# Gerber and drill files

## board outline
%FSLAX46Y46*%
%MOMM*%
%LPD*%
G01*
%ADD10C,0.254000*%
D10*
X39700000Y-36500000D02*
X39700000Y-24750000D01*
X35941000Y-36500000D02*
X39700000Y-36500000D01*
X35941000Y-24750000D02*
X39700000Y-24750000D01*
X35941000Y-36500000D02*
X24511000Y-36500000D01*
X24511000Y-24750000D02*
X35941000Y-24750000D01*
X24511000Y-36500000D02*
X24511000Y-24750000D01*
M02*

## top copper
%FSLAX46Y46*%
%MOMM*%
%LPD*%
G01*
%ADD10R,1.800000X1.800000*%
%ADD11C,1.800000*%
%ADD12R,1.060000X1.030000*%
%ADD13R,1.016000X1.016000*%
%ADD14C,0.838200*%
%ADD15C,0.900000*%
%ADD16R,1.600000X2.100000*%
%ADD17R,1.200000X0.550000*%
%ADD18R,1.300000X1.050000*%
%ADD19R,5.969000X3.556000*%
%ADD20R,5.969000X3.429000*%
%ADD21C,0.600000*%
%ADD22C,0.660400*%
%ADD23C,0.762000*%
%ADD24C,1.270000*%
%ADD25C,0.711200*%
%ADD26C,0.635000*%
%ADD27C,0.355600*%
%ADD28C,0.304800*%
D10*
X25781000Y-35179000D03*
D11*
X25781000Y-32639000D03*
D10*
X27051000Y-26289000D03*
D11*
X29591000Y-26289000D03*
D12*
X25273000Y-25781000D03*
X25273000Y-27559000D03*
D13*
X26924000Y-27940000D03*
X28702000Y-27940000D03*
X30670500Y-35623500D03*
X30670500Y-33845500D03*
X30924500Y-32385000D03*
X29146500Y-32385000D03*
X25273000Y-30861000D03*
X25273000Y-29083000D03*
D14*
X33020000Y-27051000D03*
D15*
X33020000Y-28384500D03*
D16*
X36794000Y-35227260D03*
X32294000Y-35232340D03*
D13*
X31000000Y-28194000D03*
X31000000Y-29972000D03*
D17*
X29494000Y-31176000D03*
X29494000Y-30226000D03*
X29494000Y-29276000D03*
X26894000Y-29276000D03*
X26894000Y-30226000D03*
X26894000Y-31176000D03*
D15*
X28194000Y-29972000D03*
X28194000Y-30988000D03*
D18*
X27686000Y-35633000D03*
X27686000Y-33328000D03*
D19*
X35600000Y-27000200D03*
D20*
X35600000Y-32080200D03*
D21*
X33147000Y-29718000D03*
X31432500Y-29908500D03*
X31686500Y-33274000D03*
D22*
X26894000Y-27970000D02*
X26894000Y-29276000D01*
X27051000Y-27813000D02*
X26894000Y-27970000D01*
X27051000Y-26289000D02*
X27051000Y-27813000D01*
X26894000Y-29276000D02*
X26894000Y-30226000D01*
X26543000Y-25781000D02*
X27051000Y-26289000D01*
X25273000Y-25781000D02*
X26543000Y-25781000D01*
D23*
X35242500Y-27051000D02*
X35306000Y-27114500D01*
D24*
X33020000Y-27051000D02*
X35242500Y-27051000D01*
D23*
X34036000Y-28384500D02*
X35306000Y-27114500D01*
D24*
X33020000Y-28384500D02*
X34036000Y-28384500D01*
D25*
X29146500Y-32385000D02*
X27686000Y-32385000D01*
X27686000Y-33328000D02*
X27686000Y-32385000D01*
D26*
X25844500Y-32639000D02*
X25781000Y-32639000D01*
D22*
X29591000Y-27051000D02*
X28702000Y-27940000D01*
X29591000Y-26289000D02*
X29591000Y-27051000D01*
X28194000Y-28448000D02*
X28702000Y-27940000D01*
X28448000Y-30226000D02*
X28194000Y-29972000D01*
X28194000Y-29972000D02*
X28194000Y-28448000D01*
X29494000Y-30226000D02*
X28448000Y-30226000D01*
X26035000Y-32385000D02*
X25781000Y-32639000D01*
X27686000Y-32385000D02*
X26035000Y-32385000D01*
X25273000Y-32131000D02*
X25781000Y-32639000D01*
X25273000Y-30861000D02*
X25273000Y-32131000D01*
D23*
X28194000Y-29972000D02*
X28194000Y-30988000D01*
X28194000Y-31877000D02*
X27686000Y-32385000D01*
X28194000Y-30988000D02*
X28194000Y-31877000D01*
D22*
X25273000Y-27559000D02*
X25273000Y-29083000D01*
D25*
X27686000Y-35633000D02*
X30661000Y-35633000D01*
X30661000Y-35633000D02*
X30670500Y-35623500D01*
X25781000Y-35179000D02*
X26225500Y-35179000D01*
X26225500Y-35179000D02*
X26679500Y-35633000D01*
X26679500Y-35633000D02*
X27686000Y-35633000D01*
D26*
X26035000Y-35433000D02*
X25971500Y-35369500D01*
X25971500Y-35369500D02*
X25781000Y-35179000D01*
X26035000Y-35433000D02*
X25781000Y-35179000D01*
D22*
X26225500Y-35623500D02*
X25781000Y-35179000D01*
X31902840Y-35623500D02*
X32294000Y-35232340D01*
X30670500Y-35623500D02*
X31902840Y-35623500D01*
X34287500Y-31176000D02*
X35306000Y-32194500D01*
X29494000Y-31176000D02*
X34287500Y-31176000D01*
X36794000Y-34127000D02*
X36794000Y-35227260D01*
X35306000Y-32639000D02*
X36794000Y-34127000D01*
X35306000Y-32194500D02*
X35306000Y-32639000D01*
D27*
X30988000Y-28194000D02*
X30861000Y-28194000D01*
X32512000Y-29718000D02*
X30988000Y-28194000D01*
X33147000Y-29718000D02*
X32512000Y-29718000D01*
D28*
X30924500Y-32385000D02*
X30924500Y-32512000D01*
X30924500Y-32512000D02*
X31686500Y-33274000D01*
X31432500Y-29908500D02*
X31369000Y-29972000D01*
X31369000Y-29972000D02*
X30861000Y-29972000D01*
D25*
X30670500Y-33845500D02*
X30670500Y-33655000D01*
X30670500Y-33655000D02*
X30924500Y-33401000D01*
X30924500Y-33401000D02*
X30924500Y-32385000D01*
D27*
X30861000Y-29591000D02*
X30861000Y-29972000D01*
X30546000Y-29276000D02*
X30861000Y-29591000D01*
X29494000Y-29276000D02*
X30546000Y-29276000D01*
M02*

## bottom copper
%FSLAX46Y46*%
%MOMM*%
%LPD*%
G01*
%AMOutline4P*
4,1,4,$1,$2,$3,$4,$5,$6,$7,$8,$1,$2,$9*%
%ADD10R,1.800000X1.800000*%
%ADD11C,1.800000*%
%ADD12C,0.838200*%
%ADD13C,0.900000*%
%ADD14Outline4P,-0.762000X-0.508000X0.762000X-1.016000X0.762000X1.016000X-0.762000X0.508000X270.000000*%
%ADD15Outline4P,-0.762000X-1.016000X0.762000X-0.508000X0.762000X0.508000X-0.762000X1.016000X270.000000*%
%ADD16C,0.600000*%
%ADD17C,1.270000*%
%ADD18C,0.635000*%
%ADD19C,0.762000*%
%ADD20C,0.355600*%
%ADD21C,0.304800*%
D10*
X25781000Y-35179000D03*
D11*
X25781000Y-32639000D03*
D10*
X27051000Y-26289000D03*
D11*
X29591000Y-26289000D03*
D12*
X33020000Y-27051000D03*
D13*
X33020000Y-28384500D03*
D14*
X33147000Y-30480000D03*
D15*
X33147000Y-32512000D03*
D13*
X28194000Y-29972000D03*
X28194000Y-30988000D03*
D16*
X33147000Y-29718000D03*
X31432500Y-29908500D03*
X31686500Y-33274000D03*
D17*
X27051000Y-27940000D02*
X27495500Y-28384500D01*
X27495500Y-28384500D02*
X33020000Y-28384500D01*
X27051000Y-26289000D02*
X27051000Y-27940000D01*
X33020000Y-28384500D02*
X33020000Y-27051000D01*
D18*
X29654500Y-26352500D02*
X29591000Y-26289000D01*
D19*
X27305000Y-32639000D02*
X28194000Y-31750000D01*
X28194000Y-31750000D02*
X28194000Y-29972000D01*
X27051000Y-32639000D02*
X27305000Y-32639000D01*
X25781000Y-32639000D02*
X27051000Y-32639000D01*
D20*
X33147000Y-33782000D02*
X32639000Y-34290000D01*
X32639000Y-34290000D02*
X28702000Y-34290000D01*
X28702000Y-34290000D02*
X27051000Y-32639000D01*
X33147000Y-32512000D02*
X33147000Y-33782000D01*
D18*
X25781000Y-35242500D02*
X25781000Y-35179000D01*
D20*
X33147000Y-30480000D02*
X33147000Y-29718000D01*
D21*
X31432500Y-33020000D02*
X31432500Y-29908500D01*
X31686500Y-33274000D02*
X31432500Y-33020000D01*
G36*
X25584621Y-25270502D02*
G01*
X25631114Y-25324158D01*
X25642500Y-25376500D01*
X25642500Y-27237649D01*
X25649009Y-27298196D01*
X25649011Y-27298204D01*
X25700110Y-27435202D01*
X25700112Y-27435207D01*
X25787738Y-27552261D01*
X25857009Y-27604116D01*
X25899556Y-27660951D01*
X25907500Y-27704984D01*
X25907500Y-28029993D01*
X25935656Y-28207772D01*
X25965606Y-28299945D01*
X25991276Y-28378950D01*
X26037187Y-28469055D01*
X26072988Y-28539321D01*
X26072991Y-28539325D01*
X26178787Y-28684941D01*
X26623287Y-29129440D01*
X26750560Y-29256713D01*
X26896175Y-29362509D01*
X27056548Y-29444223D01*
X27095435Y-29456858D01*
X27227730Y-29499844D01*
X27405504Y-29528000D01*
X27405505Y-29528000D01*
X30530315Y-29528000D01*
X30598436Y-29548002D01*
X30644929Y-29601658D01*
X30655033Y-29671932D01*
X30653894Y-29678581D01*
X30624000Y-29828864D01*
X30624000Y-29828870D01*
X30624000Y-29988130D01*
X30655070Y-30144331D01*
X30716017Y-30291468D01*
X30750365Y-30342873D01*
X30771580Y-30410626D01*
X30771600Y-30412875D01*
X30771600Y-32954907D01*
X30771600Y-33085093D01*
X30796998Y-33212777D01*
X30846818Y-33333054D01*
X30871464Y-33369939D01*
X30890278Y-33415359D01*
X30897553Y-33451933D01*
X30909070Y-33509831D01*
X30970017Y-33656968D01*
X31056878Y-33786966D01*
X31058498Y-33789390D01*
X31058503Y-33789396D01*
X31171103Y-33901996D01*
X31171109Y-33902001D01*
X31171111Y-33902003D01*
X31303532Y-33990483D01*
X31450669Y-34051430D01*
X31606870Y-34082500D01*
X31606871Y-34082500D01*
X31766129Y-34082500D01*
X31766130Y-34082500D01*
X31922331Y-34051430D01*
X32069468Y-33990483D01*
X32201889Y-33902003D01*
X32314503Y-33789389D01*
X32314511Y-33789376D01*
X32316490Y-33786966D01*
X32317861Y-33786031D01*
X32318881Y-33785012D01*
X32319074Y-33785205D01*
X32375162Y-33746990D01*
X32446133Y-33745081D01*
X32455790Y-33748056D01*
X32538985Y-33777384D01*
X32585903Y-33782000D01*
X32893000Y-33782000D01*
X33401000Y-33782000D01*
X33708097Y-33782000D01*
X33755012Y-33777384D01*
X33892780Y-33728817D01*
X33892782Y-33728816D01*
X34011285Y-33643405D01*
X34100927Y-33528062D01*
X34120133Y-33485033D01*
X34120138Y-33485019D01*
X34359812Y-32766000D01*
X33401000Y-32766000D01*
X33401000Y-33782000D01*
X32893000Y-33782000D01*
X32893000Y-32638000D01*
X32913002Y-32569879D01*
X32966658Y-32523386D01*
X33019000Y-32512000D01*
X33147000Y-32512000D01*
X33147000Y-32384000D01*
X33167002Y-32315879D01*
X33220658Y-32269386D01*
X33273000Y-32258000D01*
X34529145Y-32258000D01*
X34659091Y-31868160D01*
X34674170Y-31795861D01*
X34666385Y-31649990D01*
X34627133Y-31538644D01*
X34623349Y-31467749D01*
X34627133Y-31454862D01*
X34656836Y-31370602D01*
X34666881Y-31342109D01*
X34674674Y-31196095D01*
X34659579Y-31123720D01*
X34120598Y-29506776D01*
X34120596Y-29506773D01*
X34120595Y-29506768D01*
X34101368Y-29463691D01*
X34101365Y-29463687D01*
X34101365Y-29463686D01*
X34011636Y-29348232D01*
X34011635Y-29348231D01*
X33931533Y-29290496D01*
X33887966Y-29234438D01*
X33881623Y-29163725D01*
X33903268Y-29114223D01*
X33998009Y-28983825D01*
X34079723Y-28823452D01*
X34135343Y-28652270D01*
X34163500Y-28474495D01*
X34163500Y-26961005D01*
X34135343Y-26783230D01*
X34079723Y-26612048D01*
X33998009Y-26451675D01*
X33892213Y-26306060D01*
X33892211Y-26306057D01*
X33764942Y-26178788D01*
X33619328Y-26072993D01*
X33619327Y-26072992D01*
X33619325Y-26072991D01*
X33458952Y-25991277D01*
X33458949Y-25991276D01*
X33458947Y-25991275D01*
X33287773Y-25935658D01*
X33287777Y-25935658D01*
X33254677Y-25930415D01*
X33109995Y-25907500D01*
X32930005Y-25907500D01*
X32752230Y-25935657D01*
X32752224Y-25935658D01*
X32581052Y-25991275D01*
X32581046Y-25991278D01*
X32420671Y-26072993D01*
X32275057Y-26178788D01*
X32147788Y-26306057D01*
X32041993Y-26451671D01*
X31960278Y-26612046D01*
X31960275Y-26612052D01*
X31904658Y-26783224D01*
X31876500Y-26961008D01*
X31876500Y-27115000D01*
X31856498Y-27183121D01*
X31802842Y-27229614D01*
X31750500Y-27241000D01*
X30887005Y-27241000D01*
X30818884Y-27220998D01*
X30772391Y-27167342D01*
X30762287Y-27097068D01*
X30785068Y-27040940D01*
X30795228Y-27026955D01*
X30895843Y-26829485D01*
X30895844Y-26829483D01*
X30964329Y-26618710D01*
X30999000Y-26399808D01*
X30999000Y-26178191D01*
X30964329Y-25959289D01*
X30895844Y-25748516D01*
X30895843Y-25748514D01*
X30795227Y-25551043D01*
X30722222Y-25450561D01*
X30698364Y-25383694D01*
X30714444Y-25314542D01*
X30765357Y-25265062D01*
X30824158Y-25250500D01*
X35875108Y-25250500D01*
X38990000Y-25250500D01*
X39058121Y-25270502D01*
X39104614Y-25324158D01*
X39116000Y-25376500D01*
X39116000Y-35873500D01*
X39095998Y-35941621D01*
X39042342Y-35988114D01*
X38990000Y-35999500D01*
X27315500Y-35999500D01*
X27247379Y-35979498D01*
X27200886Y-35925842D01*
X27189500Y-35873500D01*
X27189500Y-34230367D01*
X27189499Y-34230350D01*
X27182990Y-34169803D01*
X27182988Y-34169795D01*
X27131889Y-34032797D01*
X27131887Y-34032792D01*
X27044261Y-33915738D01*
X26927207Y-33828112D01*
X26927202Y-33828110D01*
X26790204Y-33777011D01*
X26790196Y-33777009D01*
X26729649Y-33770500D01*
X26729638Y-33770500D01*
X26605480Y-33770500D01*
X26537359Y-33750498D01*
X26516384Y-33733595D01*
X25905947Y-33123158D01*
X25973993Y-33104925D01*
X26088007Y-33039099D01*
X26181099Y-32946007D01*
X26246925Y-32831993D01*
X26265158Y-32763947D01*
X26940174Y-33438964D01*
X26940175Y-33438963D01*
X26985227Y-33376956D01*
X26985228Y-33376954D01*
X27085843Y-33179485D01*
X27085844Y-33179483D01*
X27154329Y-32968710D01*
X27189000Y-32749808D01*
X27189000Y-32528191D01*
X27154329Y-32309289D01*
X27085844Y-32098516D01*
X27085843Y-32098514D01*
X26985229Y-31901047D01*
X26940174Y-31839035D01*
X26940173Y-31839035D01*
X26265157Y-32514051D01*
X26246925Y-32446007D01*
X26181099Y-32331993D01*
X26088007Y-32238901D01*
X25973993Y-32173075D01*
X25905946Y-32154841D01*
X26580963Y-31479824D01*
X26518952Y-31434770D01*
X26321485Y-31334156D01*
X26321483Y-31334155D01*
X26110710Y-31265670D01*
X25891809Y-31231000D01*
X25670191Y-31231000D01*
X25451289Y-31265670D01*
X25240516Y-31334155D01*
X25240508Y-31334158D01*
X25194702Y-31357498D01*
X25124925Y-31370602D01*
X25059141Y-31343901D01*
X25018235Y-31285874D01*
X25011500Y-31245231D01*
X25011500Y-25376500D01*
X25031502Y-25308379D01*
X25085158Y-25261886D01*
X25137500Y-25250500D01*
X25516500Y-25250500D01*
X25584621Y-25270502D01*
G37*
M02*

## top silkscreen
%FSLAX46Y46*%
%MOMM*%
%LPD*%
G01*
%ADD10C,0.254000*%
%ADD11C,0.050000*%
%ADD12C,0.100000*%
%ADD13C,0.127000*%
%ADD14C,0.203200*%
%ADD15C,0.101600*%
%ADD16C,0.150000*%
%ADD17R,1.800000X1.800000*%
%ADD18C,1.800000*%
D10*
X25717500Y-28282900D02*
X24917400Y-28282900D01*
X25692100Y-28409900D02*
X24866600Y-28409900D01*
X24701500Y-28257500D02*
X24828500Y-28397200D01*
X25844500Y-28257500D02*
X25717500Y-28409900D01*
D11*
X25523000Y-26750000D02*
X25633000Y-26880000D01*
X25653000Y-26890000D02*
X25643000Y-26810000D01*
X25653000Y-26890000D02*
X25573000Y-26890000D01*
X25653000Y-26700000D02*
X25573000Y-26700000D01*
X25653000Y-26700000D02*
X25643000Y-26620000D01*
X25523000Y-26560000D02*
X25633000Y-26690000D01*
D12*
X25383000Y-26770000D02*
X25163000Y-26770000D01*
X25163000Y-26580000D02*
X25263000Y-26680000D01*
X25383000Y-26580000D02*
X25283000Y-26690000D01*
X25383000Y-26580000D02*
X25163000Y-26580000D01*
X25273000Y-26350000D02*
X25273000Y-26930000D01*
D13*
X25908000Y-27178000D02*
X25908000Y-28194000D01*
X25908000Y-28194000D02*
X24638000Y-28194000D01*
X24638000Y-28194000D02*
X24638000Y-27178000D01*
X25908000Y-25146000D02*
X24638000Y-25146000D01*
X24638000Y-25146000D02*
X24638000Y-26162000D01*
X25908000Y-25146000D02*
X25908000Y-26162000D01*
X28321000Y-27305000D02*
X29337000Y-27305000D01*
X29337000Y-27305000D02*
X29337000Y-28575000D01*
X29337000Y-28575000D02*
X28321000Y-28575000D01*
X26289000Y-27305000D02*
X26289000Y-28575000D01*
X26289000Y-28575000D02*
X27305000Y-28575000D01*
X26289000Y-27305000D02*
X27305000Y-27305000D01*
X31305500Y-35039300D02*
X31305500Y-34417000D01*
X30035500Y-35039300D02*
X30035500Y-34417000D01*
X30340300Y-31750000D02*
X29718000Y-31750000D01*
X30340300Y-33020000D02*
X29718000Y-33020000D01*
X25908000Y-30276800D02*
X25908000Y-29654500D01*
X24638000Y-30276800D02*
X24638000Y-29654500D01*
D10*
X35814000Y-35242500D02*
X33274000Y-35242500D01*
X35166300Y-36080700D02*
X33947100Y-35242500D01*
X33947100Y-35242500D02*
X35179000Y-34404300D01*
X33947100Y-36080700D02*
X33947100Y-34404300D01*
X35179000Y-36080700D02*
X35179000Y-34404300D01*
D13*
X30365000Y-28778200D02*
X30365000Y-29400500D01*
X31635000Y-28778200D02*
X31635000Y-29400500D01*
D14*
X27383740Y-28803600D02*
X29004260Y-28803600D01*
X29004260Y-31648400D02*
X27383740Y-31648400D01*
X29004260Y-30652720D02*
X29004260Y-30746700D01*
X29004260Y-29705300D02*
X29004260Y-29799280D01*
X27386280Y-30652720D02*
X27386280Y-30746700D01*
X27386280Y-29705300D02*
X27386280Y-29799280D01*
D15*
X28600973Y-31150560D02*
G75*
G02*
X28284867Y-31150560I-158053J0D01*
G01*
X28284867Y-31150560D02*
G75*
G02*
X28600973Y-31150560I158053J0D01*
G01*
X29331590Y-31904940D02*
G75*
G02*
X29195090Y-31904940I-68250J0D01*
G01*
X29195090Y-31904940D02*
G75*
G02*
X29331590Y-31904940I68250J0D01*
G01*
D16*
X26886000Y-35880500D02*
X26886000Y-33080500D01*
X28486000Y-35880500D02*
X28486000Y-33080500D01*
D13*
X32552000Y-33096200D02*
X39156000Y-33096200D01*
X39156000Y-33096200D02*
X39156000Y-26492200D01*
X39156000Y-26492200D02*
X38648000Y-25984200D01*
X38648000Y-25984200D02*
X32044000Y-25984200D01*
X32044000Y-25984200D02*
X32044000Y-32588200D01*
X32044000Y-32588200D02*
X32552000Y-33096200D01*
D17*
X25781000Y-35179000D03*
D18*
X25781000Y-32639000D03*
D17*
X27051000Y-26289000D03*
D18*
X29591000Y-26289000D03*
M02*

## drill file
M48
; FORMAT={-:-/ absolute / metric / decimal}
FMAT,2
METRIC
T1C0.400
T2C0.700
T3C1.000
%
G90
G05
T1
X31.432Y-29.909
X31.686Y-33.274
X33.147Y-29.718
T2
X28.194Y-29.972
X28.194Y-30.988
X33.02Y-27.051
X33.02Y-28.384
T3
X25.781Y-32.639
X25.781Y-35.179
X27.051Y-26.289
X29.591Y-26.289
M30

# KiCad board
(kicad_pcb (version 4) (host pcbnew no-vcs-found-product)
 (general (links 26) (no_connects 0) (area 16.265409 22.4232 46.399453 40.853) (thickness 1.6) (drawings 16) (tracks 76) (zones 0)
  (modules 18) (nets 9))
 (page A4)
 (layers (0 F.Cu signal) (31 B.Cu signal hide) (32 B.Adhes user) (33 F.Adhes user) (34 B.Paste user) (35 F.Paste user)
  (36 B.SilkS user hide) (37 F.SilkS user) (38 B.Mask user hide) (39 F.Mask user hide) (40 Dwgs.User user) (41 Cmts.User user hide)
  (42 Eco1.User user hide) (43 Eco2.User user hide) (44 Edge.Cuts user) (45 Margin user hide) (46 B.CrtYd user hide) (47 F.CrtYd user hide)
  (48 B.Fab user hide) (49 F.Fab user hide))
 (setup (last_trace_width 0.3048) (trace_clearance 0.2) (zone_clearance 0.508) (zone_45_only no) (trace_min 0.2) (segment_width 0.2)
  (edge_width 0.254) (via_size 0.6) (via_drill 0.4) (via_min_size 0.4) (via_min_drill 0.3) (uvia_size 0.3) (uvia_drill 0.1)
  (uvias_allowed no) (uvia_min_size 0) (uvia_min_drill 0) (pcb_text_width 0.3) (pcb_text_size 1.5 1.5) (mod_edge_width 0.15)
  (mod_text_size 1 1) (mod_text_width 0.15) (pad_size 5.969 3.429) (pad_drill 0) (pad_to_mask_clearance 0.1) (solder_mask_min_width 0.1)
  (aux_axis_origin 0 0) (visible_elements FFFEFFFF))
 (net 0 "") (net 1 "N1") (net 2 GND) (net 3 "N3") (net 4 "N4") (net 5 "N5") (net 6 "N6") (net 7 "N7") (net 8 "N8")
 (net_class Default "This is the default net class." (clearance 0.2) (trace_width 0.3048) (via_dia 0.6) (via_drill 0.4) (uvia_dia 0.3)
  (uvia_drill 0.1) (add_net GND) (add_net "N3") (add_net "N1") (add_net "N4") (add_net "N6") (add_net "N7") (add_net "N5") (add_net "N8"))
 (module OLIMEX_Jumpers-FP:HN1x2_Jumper (layer F.Cu) (at 25.781 33.909 90)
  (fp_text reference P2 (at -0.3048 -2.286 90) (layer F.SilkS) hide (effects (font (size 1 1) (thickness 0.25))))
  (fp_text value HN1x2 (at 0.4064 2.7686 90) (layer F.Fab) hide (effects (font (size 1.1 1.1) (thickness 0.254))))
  (pad 1 thru_hole rect (at -1.27 0 180) (size 1.8 1.8) (drill 1) (layers *.Cu *.Mask F.SilkS) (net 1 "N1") (solder_mask_margin 0.0508)
   (solder_paste_margin -0.0508))
  (pad 2 thru_hole circle (at 1.27 0 180) (size 1.8 1.8) (drill 1) (layers *.Cu *.Mask F.SilkS) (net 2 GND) (solder_mask_margin 0.0508)
   (solder_paste_margin -0.0508)))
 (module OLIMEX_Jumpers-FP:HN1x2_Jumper (layer F.Cu) (at 28.321 26.289)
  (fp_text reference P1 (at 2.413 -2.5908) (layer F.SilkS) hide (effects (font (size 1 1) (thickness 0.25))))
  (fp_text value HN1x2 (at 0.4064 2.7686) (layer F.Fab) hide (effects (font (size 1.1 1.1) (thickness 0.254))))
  (pad 1 thru_hole rect (at -1.27 0 90) (size 1.8 1.8) (drill 1) (layers *.Cu *.Mask F.SilkS) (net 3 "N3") (solder_mask_margin 0.0508)
   (solder_paste_margin -0.0508))
  (pad 2 thru_hole circle (at 1.27 0 90) (size 1.8 1.8) (drill 1) (layers *.Cu *.Mask F.SilkS) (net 2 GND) (solder_mask_margin 0.0508)
   (solder_paste_margin -0.0508)))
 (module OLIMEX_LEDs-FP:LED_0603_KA (layer F.Cu) (at 25.273 26.67 270)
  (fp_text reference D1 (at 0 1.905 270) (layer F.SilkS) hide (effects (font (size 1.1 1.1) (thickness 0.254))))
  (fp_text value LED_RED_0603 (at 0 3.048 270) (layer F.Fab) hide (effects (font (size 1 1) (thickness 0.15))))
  (fp_line (start 1.6129 -0.4445) (end 1.6129 0.3556) (layer F.SilkS) (width 0.254))
  (fp_line (start 1.7399 -0.4191) (end 1.7399 0.4064) (layer F.SilkS) (width 0.254))
  (fp_line (start 1.5875 0.5715) (end 1.7272 0.4445) (layer F.SilkS) (width 0.254))
  (fp_line (start 1.5875 -0.5715) (end 1.7399 -0.4445) (layer F.SilkS) (width 0.254))
  (fp_line (start 0.08 -0.25) (end 0.21 -0.36) (layer F.SilkS) (width 0.05))
  (fp_line (start 0.22 -0.38) (end 0.14 -0.37) (layer F.SilkS) (width 0.05))
  (fp_line (start 0.22 -0.38) (end 0.22 -0.3) (layer F.SilkS) (width 0.05))
  (fp_line (start 0.03 -0.38) (end 0.03 -0.3) (layer F.SilkS) (width 0.05))
  (fp_line (start 0.03 -0.38) (end -0.05 -0.37) (layer F.SilkS) (width 0.05))
  (fp_line (start -0.11 -0.25) (end 0.02 -0.36) (layer F.SilkS) (width 0.05))
  (fp_line (start 0.1 -0.11) (end 0.1 0.11) (layer F.SilkS) (width 0.1))
  (fp_line (start -0.09 0.11) (end 0.01 0.01) (layer F.SilkS) (width 0.1))
  (fp_line (start -0.09 -0.11) (end 0.02 -0.01) (layer F.SilkS) (width 0.1))
  (fp_line (start -0.09 -0.11) (end -0.09 0.11) (layer F.SilkS) (width 0.1))
  (fp_line (start -0.32 0) (end 0.26 0) (layer F.SilkS) (width 0.1))
  (fp_line (start 0.508 -0.635) (end 1.524 -0.635) (layer F.SilkS) (width 0.127))
  (fp_line (start 1.524 -0.635) (end 1.524 0.635) (layer F.SilkS) (width 0.127))
  (fp_line (start 1.524 0.635) (end 0.508 0.635) (layer F.SilkS) (width 0.127))
  (fp_line (start -1.524 -0.635) (end -1.524 0.635) (layer F.SilkS) (width 0.127))
  (fp_line (start -1.524 0.635) (end -0.508 0.635) (layer F.SilkS) (width 0.127))
  (fp_line (start -1.524 -0.635) (end -0.508 -0.635) (layer F.SilkS) (width 0.127))
  (pad 2 smd rect (at -0.889 0 270) (size 1.03 1.06) (layers F.Cu F.Paste F.Mask) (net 3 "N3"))
  (pad 1 smd rect (at 0.889 0 270) (size 1.03 1.06) (layers F.Cu F.Paste F.Mask) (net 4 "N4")))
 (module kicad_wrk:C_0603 (layer F.Cu) (at 27.813 27.94)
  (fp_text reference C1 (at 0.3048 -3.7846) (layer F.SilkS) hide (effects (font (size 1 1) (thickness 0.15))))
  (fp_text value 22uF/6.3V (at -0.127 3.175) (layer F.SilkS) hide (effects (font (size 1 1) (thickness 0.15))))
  (fp_line (start 0.508 -0.635) (end 1.524 -0.635) (layer F.SilkS) (width 0.127))
  (fp_line (start 1.524 -0.635) (end 1.524 0.635) (layer F.SilkS) (width 0.127))
  (fp_line (start 1.524 0.635) (end 0.508 0.635) (layer F.SilkS) (width 0.127))
  (fp_line (start -1.524 -0.635) (end -1.524 0.635) (layer F.SilkS) (width 0.127))
  (fp_line (start -1.524 0.635) (end -0.508 0.635) (layer F.SilkS) (width 0.127))
  (fp_line (start -1.524 -0.635) (end -0.508 -0.635) (layer F.SilkS) (width 0.127))
  (pad 1 smd rect (at -0.889 0) (size 1.016 1.016) (layers F.Cu F.Paste F.Mask) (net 3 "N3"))
  (pad 2 smd rect (at 0.889 0) (size 1.016 1.016) (layers F.Cu F.Paste F.Mask) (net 2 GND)))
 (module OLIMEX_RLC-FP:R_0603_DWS (layer F.Cu) (at 30.6705 34.7345 90)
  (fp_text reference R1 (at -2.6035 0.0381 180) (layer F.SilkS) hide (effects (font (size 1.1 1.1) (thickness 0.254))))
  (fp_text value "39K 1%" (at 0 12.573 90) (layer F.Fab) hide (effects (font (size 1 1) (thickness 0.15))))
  (fp_line (start -0.3048 0.635) (end 0.3175 0.635) (layer F.SilkS) (width 0.127))
  (fp_line (start -0.3048 -0.635) (end 0.3175 -0.635) (layer F.SilkS) (width 0.127))
  (pad 1 smd rect (at -0.889 0 90) (size 1.016 1.016) (layers F.Cu F.Paste F.Mask) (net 1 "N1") (solder_mask_margin 0.0508)
   (solder_paste_margin -0.0508) (clearance 0.0508))
  (pad 2 smd rect (at 0.889 0 90) (size 1.016 1.016) (layers F.Cu F.Paste F.Mask) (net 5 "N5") (solder_mask_margin 0.0508)
   (solder_paste_margin -0.0508) (clearance 0.0508)))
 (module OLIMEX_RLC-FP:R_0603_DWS (layer F.Cu) (at 30.0355 32.385 180)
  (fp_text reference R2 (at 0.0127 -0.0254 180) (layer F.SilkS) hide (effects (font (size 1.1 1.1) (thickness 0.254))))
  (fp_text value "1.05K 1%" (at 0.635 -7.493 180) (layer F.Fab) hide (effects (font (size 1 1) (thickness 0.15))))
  (fp_line (start -0.3048 0.635) (end 0.3175 0.635) (layer F.SilkS) (width 0.127))
  (fp_line (start -0.3048 -0.635) (end 0.3175 -0.635) (layer F.SilkS) (width 0.127))
  (pad 1 smd rect (at -0.889 0 180) (size 1.016 1.016) (layers F.Cu F.Paste F.Mask) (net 5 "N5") (solder_mask_margin 0.0508)
   (solder_paste_margin -0.0508) (clearance 0.0508))
  (pad 2 smd rect (at 0.889 0 180) (size 1.016 1.016) (layers F.Cu F.Paste F.Mask) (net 2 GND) (solder_mask_margin 0.0508)
   (solder_paste_margin -0.0508) (clearance 0.0508)))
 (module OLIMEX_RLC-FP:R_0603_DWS (layer F.Cu) (at 25.273 29.972 90)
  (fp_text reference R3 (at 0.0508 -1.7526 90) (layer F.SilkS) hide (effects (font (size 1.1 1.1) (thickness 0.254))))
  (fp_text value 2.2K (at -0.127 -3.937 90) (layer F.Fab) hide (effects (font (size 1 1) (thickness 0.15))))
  (fp_line (start -0.3048 0.635) (end 0.3175 0.635) (layer F.SilkS) (width 0.127))
  (fp_line (start -0.3048 -0.635) (end 0.3175 -0.635) (layer F.SilkS) (width 0.127))
  (pad 1 smd rect (at -0.889 0 90) (size 1.016 1.016) (layers F.Cu F.Paste F.Mask) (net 2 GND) (solder_mask_margin 0.0508)
   (solder_paste_margin -0.0508) (clearance 0.0508))
  (pad 2 smd rect (at 0.889 0 90) (size 1.016 1.016) (layers F.Cu F.Paste F.Mask) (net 4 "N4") (solder_mask_margin 0.0508)
   (solder_paste_margin -0.0508) (clearance 0.0508)))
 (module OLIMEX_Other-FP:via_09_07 (layer F.Cu) (at 33.02 27.051 180)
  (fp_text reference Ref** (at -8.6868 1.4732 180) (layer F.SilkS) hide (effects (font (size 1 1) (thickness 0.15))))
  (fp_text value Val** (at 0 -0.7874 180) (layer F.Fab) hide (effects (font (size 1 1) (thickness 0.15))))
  (pad 0 thru_hole circle (at 0 0 180) (size 0.8382 0.8382) (drill 0.7) (layers *.Cu) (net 3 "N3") (zone_connect 2)))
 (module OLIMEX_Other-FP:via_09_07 (layer F.Cu) (at 33.02 28.321 180)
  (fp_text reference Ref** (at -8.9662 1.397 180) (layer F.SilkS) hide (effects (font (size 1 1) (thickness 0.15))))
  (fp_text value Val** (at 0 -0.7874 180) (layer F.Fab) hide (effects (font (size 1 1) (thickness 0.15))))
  (pad 0 thru_hole circle (at 0 -0.0635 180) (size 0.9 0.9) (drill 0.7) (layers *.Cu) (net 3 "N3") (zone_connect 2)))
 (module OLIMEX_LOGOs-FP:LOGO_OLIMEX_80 (layer B.Cu) (at 35.8775 27.686 180)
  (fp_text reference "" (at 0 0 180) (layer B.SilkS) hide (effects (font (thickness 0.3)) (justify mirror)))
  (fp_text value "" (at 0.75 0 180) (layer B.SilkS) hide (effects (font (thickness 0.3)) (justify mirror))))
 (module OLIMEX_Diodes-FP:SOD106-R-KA (layer F.Cu) (at 34.544 35.2425 180)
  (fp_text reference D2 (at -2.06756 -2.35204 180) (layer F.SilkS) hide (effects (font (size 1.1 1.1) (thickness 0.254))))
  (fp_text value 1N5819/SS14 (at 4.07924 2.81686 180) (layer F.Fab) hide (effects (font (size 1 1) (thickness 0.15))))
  (fp_line (start -1.27 0) (end 1.27 0) (layer F.SilkS) (width 0.254))
  (fp_line (start -0.6223 -0.8382) (end 0.5969 0) (layer F.SilkS) (width 0.254))
  (fp_line (start 0.5969 0) (end -0.635 0.8382) (layer F.SilkS) (width 0.254))
  (fp_line (start 0.5969 -0.8382) (end 0.5969 0.8382) (layer F.SilkS) (width 0.254))
  (fp_line (start -0.635 -0.8382) (end -0.635 0.8382) (layer F.SilkS) (width 0.254))
  (pad 2 smd rect (at -2.25 0.01524 180) (size 1.6 2.1) (layers F.Cu F.Paste F.Mask) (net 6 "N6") (solder_mask_margin 0.0508)
   (solder_paste_margin -0.0508) (clearance 0.0508))
  (pad 1 smd rect (at 2.25 0.01016 180) (size 1.6 2.1) (layers F.Cu F.Paste F.Mask) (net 1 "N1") (solder_mask_margin 0.0508)
   (solder_paste_margin -0.0508) (clearance 0.0508)))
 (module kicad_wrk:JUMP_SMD (layer B.Cu) (at 33.147 31.496 270)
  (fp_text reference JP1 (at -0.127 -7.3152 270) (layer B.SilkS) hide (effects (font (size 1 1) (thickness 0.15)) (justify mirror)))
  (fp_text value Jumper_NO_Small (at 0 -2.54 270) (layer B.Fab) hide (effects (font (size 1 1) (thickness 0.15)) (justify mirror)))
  (pad 1 smd trapezoid (at -1.016 0 270) (size 1.524 1.524) (rect_delta -0.508 0) (layers B.Cu B.Mask) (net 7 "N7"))
  (pad 2 smd trapezoid (at 1.016 0 270) (size 1.524 1.524) (rect_delta 0.508 0) (layers B.Cu B.Mask) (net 2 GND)))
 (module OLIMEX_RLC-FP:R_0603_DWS (layer F.Cu) (at 31 29.083 270)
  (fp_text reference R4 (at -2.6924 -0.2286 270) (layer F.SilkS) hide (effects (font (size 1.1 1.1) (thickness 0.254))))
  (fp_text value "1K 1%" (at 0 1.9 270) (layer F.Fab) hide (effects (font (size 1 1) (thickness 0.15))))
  (fp_line (start -0.3048 0.635) (end 0.3175 0.635) (layer F.SilkS) (width 0.127))
  (fp_line (start -0.3048 -0.635) (end 0.3175 -0.635) (layer F.SilkS) (width 0.127))
  (pad 1 smd rect (at -0.889 0 270) (size 1.016 1.016) (layers F.Cu F.Paste F.Mask) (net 7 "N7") (solder_mask_margin 0.0508)
   (solder_paste_margin -0.0508) (clearance 0.0508))
  (pad 2 smd rect (at 0.889 0 270) (size 1.016 1.016) (layers F.Cu F.Paste F.Mask) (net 5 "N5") (solder_mask_margin 0.0508)
   (solder_paste_margin -0.0508) (clearance 0.0508)))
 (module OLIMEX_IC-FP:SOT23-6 (layer F.Cu) (at 28.194 30.226)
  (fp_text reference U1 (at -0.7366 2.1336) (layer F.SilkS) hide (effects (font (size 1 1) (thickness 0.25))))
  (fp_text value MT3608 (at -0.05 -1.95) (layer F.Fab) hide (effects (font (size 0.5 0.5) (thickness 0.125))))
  (fp_line (start -0.81026 -1.4224) (end 0.81026 -1.4224) (layer F.SilkS) (width 0.2032))
  (fp_line (start 0.81026 1.4224) (end -0.81026 1.4224) (layer F.SilkS) (width 0.2032))
  (fp_line (start 0.81026 0.42672) (end 0.81026 0.5207) (layer F.SilkS) (width 0.2032))
  (fp_line (start 0.81026 -0.5207) (end 0.81026 -0.42672) (layer F.SilkS) (width 0.2032))
  (fp_line (start -0.80772 0.42672) (end -0.80772 0.5207) (layer F.SilkS) (width 0.2032))
  (fp_line (start -0.80772 -0.5207) (end -0.80772 -0.42672) (layer F.SilkS) (width 0.2032))
  (fp_circle (center 0.24892 0.92456) (end 0.36068 1.03632) (layer F.SilkS) (width 0.1016))
  (fp_circle (center 1.06934 1.67894) (end 1.1176 1.7272) (layer F.SilkS) (width 0.1016))
  (pad 1 smd rect (at 1.3 0.95 90) (size 0.55 1.2) (layers F.Cu F.Paste F.Mask) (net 6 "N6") (solder_mask_margin 0.0508)
   (solder_paste_margin -0.0508) (clearance 0.0508))
  (pad 2 smd rect (at 1.3 0 90) (size 0.55 1.2) (layers F.Cu F.Paste F.Mask) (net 2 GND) (solder_mask_margin 0.0508)
   (solder_paste_margin -0.0508) (clearance 0.0508))
  (pad 3 smd rect (at 1.3 -0.95 90) (size 0.55 1.2) (layers F.Cu F.Paste F.Mask) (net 5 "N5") (solder_mask_margin 0.0508)
   (solder_paste_margin -0.0508) (clearance 0.0508))
  (pad 4 smd rect (at -1.3 -0.95 90) (size 0.55 1.2) (layers F.Cu F.Paste F.Mask) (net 3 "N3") (solder_mask_margin 0.0508)
   (solder_paste_margin -0.0508) (clearance 0.0508))
  (pad 5 smd rect (at -1.3 0 90) (size 0.55 1.2) (layers F.Cu F.Paste F.Mask) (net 3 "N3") (solder_mask_margin 0.0508)
   (solder_paste_margin -0.0508) (clearance 0.0508))
  (pad 6 smd rect (at -1.3 0.95 90) (size 0.55 1.2) (layers F.Cu F.Paste F.Mask) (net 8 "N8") (solder_mask_margin 0.0508)
   (solder_paste_margin -0.0508) (clearance 0.0508)))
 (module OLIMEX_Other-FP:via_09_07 (layer F.Cu) (at 28.194 29.972)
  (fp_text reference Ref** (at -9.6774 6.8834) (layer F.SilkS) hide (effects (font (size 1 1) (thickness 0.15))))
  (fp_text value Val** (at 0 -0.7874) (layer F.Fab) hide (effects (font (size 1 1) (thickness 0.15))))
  (pad 0 thru_hole circle (at 0 0) (size 0.9 0.9) (drill 0.7) (layers *.Cu) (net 2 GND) (zone_connect 2)))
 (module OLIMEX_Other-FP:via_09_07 (layer F.Cu) (at 28.194 30.988)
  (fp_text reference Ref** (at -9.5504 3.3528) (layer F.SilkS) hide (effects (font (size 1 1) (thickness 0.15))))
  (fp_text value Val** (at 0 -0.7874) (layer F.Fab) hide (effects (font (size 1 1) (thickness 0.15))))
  (pad 0 thru_hole circle (at 0 0) (size 0.9 0.9) (drill 0.7) (layers *.Cu) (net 2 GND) (zone_connect 2)))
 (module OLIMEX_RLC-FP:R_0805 (layer F.Cu) (at 27.686 34.4805 180)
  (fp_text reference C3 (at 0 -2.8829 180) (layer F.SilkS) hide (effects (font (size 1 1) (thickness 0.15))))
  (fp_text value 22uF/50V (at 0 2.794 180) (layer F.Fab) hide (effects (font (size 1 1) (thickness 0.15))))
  (fp_line (start 0.8 -1.4) (end 0.8 1.4) (layer F.SilkS) (width 0.15))
  (fp_line (start -0.8 -1.4) (end -0.8 1.4) (layer F.SilkS) (width 0.15))
  (pad 1 smd rect (at 0 -1.1525 180) (size 1.3 1.05) (layers F.Cu F.Paste F.Mask) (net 1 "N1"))
  (pad 2 smd rect (at 0 1.1525 180) (size 1.3 1.05) (layers F.Cu F.Paste F.Mask) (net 2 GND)))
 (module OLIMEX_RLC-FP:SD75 (layer F.Cu) (at 35.6 29.5402)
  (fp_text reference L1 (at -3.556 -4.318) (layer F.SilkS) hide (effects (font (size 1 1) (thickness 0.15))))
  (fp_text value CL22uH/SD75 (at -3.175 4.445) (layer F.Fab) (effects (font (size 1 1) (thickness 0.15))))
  (fp_line (start -3.048 3.556) (end 3.556 3.556) (layer F.SilkS) (width 0.127))
  (fp_line (start 3.556 3.556) (end 3.556 -3.048) (layer F.SilkS) (width 0.127))
  (fp_line (start 3.556 -3.048) (end 3.048 -3.556) (layer F.SilkS) (width 0.127))
  (fp_line (start 3.048 -3.556) (end -3.556 -3.556) (layer F.SilkS) (width 0.127))
  (fp_line (start -3.556 -3.556) (end -3.556 3.048) (layer F.SilkS) (width 0.127))
  (fp_line (start -3.556 3.048) (end -3.048 3.556) (layer F.SilkS) (width 0.127))
  (pad 1 smd rect (at 0 -2.54) (size 5.969 3.556) (layers F.Cu F.Paste F.Mask) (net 3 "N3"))
  (pad 2 smd rect (at 0 2.54) (size 5.969 3.429) (layers F.Cu F.Paste F.Mask) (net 6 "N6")))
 (gr_line (start 39.7 36.5) (end 39.7 24.75) (angle 90) (layer Edge.Cuts) (width 0.254))
 (gr_line (start 35.941 36.5) (end 39.7 36.5) (angle 90) (layer Edge.Cuts) (width 0.254))
 (gr_line (start 35.941 24.75) (end 39.7 24.75) (angle 90) (layer Edge.Cuts) (width 0.254))
 (gr_line (start 35.941 36.5) (end 24.511 36.5) (angle 90) (layer Edge.Cuts) (width 0.254))
 (gr_line (start 24.511 24.75) (end 35.941 24.75) (angle 90) (layer Edge.Cuts) (width 0.254))
 (gr_line (start 24.511 36.5) (end 24.511 24.75) (angle 90) (layer Edge.Cuts) (width 0.254))
 (segment (start 26.894 27.97) (end 26.894 29.276) (width 0.6604) (layer F.Cu) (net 3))
 (segment (start 27.051 27.813) (end 26.894 27.97) (width 0.6604) (layer F.Cu) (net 3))
 (segment (start 27.051 26.289) (end 27.051 27.813) (width 0.6604) (layer F.Cu) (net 3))
 (segment (start 26.894 29.276) (end 26.894 30.226) (width 0.6604) (layer F.Cu) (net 3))
 (segment (start 26.543 25.781) (end 27.051 26.289) (width 0.6604) (layer F.Cu) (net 3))
 (segment (start 25.273 25.781) (end 26.543 25.781) (width 0.6604) (layer F.Cu) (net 3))
 (segment (start 35.2425 27.051) (end 35.306 27.1145) (width 0.762) (layer F.Cu) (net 3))
 (segment (start 33.02 27.051) (end 35.2425 27.051) (width 1.27) (layer F.Cu) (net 3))
 (segment (start 34.036 28.3845) (end 35.306 27.1145) (width 0.762) (layer F.Cu) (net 3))
 (segment (start 33.02 28.3845) (end 34.036 28.3845) (width 1.27) (layer F.Cu) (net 3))
 (segment (start 27.051 27.94) (end 27.4955 28.3845) (width 1.27) (layer B.Cu) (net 3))
 (segment (start 27.4955 28.3845) (end 33.02 28.3845) (width 1.27) (layer B.Cu) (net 3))
 (segment (start 27.051 26.289) (end 27.051 27.94) (width 1.27) (layer B.Cu) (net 3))
 (segment (start 33.02 28.3845) (end 33.02 27.051) (width 1.27) (layer B.Cu) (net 3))
 (segment (start 29.1465 32.385) (end 27.686 32.385) (width 0.7112) (layer F.Cu) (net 2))
 (segment (start 27.686 33.328) (end 27.686 32.385) (width 0.7112) (layer F.Cu) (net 2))
 (segment (start 29.6545 26.3525) (end 29.591 26.289) (width 0.635) (layer B.Cu) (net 2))
 (segment (start 25.8445 32.639) (end 25.781 32.639) (width 0.635) (layer F.Cu) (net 2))
 (segment (start 29.591 27.051) (end 28.702 27.94) (width 0.6604) (layer F.Cu) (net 2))
 (segment (start 29.591 26.289) (end 29.591 27.051) (width 0.6604) (layer F.Cu) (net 2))
 (segment (start 28.194 28.448) (end 28.702 27.94) (width 0.6604) (layer F.Cu) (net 2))
 (segment (start 28.448 30.226) (end 28.194 29.972) (width 0.6604) (layer F.Cu) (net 2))
 (segment (start 28.194 29.972) (end 28.194 28.448) (width 0.6604) (layer F.Cu) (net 2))
 (segment (start 29.494 30.226) (end 28.448 30.226) (width 0.6604) (layer F.Cu) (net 2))
 (segment (start 26.035 32.385) (end 25.781 32.639) (width 0.6604) (layer F.Cu) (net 2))
 (segment (start 27.686 32.385) (end 26.035 32.385) (width 0.6604) (layer F.Cu) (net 2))
 (segment (start 25.273 32.131) (end 25.781 32.639) (width 0.6604) (layer F.Cu) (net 2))
 (segment (start 25.273 30.861) (end 25.273 32.131) (width 0.6604) (layer F.Cu) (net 2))
 (segment (start 28.194 29.972) (end 28.194 30.988) (width 0.762) (layer F.Cu) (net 2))
 (segment (start 28.194 31.877) (end 27.686 32.385) (width 0.762) (layer F.Cu) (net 2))
 (segment (start 28.194 30.988) (end 28.194 31.877) (width 0.762) (layer F.Cu) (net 2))
 (segment (start 27.305 32.639) (end 28.194 31.75) (width 0.762) (layer B.Cu) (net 2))
 (segment (start 28.194 31.75) (end 28.194 29.972) (width 0.762) (layer B.Cu) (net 2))
 (segment (start 27.051 32.639) (end 27.305 32.639) (width 0.762) (layer B.Cu) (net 2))
 (segment (start 25.781 32.639) (end 27.051 32.639) (width 0.762) (layer B.Cu) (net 2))
 (segment (start 33.147 33.782) (end 32.639 34.29) (width 0.3556) (layer B.Cu) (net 2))
 (segment (start 32.639 34.29) (end 28.702 34.29) (width 0.3556) (layer B.Cu) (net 2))
 (segment (start 28.702 34.29) (end 27.051 32.639) (width 0.3556) (layer B.Cu) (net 2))
 (segment (start 33.147 32.512) (end 33.147 33.782) (width 0.3556) (layer B.Cu) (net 2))
 (segment (start 25.273 27.559) (end 25.273 29.083) (width 0.6604) (layer F.Cu) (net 4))
 (segment (start 27.686 35.633) (end 30.661 35.633) (width 0.7112) (layer F.Cu) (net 1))
 (segment (start 30.661 35.633) (end 30.6705 35.6235) (width 0.7112) (layer F.Cu) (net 1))
 (segment (start 25.781 35.179) (end 26.2255 35.179) (width 0.7112) (layer F.Cu) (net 1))
 (segment (start 26.2255 35.179) (end 26.6795 35.633) (width 0.7112) (layer F.Cu) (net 1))
 (segment (start 26.6795 35.633) (end 27.686 35.633) (width 0.7112) (layer F.Cu) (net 1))
 (segment (start 25.781 35.2425) (end 25.781 35.179) (width 0.635) (layer B.Cu) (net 1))
 (segment (start 26.035 35.433) (end 25.9715 35.3695) (width 0.635) (layer F.Cu) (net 1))
 (segment (start 25.9715 35.3695) (end 25.781 35.179) (width 0.635) (layer F.Cu) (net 1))
 (segment (start 26.035 35.433) (end 25.781 35.179) (width 0.635) (layer F.Cu) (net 1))
 (segment (start 26.2255 35.6235) (end 25.781 35.179) (width 0.6604) (layer F.Cu) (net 1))
 (segment (start 31.90284 35.6235) (end 32.294 35.23234) (width 0.6604) (layer F.Cu) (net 1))
 (segment (start 30.6705 35.6235) (end 31.90284 35.6235) (width 0.6604) (layer F.Cu) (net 1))
 (segment (start 34.2875 31.176) (end 35.306 32.1945) (width 0.6604) (layer F.Cu) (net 6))
 (segment (start 29.494 31.176) (end 34.2875 31.176) (width 0.6604) (layer F.Cu) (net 6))
 (segment (start 36.794 34.127) (end 36.794 35.22726) (width 0.6604) (layer F.Cu) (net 6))
 (segment (start 35.306 32.639) (end 36.794 34.127) (width 0.6604) (layer F.Cu) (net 6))
 (segment (start 35.306 32.1945) (end 35.306 32.639) (width 0.6604) (layer F.Cu) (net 6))
 (segment (start 30.988 28.194) (end 30.861 28.194) (width 0.3556) (layer F.Cu) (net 7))
 (segment (start 32.512 29.718) (end 30.988 28.194) (width 0.3556) (layer F.Cu) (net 7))
 (segment (start 33.147 29.718) (end 32.512 29.718) (width 0.3556) (layer F.Cu) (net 7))
 (via (at 33.147 29.718) (size 0.6) (layers F.Cu B.Cu) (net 7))
 (segment (start 33.147 30.48) (end 33.147 29.718) (width 0.3556) (layer B.Cu) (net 7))
 (segment (start 30.9245 32.385) (end 30.9245 32.512) (width 0.3048) (layer F.Cu) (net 5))
 (segment (start 30.9245 32.512) (end 31.6865 33.274) (width 0.3048) (layer F.Cu) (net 5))
 (segment (start 31.4325 29.9085) (end 31.369 29.972) (width 0.3048) (layer F.Cu) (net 5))
 (via (at 31.4325 29.9085) (size 0.6) (layers F.Cu B.Cu) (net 5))
 (segment (start 31.4325 33.02) (end 31.4325 29.9085) (width 0.3048) (layer B.Cu) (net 5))
 (segment (start 31.6865 33.274) (end 31.4325 33.02) (width 0.3048) (layer B.Cu) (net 5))
 (via (at 31.6865 33.274) (size 0.6) (layers F.Cu B.Cu) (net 5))
 (segment (start 31.369 29.972) (end 30.861 29.972) (width 0.3048) (layer F.Cu) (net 5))
 (segment (start 30.6705 33.8455) (end 30.6705 33.655) (width 0.7112) (layer F.Cu) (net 5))
 (segment (start 30.6705 33.655) (end 30.9245 33.401) (width 0.7112) (layer F.Cu) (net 5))
 (segment (start 30.9245 33.401) (end 30.9245 32.385) (width 0.7112) (layer F.Cu) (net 5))
 (segment (start 30.861 29.591) (end 30.861 29.972) (width 0.3556) (layer F.Cu) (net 5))
 (segment (start 30.546 29.276) (end 30.861 29.591) (width 0.3556) (layer F.Cu) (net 5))
 (segment (start 29.494 29.276) (end 30.546 29.276) (width 0.3556) (layer F.Cu) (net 5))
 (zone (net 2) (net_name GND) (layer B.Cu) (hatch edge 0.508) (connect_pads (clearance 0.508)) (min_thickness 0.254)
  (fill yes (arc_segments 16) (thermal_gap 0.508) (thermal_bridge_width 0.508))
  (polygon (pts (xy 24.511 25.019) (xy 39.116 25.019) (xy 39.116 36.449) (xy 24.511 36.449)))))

